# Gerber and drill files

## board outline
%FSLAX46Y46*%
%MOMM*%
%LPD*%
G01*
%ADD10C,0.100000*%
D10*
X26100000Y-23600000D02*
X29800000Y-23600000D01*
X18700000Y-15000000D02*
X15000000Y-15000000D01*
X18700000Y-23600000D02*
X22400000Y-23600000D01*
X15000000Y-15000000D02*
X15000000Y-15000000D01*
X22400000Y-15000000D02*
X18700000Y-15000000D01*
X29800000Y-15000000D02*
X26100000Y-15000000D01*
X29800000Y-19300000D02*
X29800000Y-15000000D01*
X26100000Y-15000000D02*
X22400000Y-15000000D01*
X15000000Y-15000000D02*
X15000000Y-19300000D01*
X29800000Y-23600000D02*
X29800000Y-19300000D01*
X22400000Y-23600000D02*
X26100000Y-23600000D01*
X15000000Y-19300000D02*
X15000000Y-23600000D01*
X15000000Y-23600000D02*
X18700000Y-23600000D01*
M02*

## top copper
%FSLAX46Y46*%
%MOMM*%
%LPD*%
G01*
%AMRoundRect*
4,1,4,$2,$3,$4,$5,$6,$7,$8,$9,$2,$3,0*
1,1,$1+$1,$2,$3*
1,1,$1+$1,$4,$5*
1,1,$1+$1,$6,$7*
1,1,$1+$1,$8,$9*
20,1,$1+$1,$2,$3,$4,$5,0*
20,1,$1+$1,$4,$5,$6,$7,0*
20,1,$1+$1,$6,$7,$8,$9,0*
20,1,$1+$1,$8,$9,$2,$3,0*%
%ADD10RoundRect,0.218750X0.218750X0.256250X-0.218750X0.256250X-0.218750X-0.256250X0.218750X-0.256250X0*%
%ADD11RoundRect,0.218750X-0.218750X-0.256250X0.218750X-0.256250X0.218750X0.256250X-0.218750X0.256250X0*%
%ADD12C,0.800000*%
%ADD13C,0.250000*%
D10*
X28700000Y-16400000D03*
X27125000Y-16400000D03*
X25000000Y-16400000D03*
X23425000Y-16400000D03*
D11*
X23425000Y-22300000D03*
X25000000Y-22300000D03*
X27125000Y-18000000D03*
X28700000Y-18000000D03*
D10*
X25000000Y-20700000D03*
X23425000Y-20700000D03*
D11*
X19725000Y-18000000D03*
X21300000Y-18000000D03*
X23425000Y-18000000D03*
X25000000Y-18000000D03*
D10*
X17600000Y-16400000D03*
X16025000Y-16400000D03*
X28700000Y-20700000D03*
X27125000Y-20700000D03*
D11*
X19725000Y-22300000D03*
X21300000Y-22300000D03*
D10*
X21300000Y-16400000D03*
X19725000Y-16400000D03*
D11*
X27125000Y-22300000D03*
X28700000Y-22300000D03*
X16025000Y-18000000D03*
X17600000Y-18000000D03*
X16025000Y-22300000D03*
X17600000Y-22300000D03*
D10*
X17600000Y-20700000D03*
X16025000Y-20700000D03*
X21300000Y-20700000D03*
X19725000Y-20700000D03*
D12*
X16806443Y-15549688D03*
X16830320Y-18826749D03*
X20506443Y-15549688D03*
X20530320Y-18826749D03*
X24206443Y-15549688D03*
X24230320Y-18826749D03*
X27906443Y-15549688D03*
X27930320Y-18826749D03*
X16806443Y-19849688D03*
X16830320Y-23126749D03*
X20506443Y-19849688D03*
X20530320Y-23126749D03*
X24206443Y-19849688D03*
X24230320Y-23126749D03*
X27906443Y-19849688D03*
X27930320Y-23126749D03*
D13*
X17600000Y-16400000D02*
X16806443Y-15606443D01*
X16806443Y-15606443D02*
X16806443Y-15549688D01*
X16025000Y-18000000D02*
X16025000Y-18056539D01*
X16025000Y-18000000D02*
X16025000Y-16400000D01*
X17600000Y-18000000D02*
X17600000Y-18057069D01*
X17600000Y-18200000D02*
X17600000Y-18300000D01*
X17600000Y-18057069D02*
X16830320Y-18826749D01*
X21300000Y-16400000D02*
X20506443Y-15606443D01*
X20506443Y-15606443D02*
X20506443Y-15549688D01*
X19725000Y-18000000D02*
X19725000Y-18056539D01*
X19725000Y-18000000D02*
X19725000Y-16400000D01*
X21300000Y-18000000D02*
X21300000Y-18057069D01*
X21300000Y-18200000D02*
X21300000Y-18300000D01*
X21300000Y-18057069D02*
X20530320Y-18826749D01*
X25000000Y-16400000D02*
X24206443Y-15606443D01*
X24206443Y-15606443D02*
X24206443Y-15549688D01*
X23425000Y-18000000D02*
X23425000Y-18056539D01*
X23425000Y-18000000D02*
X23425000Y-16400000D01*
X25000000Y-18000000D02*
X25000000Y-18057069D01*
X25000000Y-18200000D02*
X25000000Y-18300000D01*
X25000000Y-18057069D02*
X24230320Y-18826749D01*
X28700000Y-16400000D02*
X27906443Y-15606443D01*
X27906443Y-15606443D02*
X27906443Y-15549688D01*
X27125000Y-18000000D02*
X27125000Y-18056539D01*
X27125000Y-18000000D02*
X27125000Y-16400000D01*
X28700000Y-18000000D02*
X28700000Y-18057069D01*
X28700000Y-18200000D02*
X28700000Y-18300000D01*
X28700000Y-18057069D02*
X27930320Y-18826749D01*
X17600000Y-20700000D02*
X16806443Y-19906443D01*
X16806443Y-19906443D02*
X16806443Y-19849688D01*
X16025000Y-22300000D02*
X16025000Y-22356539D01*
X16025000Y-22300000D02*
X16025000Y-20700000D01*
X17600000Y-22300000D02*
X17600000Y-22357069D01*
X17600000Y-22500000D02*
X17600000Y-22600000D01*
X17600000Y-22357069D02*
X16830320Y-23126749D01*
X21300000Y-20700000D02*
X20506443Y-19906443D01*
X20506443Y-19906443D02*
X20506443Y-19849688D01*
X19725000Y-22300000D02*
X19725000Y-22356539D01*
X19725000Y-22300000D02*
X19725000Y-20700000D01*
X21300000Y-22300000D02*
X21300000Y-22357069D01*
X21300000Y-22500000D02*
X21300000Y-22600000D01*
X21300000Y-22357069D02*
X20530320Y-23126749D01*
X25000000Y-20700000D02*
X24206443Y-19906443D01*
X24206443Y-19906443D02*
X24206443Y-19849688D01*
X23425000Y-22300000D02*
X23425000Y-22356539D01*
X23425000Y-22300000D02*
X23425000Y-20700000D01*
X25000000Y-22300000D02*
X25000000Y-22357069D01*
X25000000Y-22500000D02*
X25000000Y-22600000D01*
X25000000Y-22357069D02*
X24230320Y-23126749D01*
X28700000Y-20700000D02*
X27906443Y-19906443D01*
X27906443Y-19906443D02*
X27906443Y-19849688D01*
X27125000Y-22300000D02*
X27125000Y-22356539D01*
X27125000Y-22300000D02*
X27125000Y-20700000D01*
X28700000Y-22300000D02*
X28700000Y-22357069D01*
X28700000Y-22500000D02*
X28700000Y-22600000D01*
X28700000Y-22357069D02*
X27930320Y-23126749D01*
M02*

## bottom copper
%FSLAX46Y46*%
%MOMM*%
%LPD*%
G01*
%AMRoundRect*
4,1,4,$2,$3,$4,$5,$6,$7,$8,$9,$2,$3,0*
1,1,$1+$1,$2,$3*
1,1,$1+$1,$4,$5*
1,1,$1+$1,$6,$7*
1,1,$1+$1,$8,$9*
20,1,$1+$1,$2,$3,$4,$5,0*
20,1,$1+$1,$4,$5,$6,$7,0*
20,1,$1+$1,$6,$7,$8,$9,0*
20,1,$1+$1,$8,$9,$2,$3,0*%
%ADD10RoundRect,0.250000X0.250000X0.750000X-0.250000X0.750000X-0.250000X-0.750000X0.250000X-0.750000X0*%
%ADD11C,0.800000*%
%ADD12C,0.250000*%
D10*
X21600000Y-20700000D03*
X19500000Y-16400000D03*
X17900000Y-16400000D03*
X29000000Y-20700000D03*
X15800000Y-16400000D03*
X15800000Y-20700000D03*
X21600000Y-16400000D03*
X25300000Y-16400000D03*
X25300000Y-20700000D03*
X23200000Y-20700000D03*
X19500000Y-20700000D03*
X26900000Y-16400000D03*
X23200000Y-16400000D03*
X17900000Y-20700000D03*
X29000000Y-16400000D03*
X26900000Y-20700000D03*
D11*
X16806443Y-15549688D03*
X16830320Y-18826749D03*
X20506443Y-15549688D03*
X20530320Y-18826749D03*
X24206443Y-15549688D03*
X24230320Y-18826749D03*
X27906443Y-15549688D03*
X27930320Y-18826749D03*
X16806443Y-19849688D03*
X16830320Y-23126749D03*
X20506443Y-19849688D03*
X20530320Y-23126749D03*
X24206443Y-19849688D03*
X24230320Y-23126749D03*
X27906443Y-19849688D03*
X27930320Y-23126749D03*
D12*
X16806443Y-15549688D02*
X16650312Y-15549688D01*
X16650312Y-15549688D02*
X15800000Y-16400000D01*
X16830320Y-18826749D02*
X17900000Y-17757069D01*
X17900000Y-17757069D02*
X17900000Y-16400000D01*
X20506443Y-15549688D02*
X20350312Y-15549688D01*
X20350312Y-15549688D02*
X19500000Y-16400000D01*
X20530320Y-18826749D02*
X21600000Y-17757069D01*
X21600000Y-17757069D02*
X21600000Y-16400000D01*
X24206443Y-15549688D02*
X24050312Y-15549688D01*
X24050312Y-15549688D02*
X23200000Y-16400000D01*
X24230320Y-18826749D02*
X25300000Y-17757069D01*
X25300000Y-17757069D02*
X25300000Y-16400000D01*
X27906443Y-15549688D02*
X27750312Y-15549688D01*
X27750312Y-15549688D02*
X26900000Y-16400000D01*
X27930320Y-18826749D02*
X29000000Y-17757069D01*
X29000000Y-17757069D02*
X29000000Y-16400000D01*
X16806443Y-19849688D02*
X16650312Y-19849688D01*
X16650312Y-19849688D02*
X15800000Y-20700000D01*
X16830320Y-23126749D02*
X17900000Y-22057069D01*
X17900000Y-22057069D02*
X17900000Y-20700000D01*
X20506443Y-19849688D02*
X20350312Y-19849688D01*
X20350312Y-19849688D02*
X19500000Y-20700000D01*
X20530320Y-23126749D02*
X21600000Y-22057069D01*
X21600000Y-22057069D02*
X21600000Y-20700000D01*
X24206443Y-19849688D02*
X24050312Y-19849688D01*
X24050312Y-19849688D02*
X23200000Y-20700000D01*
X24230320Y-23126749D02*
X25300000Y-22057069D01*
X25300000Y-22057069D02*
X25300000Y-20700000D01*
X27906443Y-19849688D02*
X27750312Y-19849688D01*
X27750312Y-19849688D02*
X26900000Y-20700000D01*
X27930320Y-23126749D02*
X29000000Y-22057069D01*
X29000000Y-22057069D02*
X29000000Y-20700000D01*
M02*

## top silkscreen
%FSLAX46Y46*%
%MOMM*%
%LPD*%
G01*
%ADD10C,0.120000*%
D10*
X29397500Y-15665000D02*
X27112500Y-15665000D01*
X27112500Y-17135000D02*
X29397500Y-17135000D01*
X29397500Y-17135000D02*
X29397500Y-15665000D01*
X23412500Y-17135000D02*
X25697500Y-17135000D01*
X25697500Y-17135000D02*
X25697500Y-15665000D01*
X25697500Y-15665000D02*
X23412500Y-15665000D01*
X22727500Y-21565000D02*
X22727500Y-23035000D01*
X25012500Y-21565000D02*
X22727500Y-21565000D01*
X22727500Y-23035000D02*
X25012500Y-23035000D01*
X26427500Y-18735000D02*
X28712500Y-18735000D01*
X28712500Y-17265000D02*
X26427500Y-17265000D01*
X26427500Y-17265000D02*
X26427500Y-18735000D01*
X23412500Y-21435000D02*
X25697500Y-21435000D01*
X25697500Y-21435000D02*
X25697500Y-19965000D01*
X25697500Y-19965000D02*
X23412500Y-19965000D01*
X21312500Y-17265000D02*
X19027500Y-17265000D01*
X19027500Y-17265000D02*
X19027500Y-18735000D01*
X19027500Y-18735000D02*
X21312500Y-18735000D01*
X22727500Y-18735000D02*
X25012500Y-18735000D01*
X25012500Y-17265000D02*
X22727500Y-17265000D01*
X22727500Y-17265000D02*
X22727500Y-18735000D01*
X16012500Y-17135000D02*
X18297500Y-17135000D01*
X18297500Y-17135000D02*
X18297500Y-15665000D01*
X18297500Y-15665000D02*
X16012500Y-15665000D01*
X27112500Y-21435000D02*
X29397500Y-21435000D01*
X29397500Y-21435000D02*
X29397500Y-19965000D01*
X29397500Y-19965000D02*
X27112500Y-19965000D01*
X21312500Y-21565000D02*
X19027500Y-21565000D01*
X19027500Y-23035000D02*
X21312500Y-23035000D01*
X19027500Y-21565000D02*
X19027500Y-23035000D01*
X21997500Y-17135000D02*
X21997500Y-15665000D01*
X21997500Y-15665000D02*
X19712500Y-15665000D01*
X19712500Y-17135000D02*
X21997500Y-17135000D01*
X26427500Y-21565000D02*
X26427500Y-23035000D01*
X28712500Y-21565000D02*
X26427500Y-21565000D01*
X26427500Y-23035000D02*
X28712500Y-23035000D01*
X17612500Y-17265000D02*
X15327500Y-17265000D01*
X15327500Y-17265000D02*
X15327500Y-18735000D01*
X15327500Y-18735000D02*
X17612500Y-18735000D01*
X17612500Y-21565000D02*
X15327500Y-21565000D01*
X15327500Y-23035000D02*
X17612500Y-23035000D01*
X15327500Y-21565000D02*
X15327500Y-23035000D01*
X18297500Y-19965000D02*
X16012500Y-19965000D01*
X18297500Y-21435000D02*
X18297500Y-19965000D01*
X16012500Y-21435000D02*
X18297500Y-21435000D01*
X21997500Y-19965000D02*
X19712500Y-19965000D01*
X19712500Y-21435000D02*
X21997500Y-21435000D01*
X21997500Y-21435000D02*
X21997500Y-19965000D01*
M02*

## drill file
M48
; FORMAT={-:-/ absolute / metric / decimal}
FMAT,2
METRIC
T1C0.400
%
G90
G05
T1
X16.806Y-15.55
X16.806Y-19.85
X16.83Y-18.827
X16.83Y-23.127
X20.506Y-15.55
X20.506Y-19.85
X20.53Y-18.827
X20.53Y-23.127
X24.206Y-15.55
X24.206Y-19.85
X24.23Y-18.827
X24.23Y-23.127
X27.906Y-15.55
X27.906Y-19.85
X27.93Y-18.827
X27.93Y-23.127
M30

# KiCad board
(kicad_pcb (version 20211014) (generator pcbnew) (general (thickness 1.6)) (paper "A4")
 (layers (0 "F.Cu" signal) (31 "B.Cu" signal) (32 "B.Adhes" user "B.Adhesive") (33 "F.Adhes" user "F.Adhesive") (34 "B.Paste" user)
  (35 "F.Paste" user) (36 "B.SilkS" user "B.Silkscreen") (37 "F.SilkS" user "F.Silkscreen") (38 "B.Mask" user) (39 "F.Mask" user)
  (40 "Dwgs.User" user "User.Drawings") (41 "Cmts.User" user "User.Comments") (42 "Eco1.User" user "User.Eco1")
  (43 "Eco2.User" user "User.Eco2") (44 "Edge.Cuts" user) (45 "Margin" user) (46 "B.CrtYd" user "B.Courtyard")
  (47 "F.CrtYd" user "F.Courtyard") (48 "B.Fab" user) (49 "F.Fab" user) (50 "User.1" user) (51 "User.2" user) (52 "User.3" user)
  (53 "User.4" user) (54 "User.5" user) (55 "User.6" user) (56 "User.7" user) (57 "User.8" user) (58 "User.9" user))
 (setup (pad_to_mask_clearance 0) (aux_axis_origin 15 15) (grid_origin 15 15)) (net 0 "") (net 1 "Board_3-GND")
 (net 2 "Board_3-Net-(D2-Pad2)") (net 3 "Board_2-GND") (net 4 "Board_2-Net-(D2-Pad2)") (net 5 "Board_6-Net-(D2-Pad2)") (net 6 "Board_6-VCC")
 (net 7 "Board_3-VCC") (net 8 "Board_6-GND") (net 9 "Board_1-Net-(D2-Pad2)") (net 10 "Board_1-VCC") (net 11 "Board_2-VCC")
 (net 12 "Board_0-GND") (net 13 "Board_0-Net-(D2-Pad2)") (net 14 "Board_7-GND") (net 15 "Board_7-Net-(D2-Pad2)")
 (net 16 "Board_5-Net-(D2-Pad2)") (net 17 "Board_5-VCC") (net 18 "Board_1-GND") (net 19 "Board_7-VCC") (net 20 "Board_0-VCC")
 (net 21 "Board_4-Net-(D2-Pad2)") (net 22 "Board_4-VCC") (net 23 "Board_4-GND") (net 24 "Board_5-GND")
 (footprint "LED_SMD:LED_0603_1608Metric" (layer "F.Cu") (at 27.9125 16.4 180)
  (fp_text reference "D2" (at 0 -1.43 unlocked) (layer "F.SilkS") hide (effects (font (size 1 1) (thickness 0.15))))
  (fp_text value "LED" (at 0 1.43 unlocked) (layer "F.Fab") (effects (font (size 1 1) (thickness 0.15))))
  (fp_line (start -1.485 0.735) (end 0.8 0.735) (layer "F.SilkS") (width 0.12))
  (fp_line (start 0.8 -0.735) (end -1.485 -0.735) (layer "F.SilkS") (width 0.12))
  (fp_line (start -1.485 -0.735) (end -1.485 0.735) (layer "F.SilkS") (width 0.12))
  (pad "1" smd roundrect (at -0.7875 0 180) (size 0.875 0.95) (layers "F.Cu" "F.Paste" "F.Mask") (roundrect_rratio 0.25)
   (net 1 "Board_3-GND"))
  (pad "2" smd roundrect (at 0.7875 0 180) (size 0.875 0.95) (layers "F.Cu" "F.Paste" "F.Mask") (roundrect_rratio 0.25)
   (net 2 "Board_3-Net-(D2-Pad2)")))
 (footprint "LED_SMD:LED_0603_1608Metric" (layer "F.Cu") (at 24.2125 16.4 180)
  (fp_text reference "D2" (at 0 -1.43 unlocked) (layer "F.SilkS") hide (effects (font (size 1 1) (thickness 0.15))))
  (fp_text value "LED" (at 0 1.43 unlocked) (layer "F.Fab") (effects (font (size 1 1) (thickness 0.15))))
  (fp_line (start 0.8 -0.735) (end -1.485 -0.735) (layer "F.SilkS") (width 0.12))
  (fp_line (start -1.485 -0.735) (end -1.485 0.735) (layer "F.SilkS") (width 0.12))
  (fp_line (start -1.485 0.735) (end 0.8 0.735) (layer "F.SilkS") (width 0.12))
  (pad "1" smd roundrect (at -0.7875 0 180) (size 0.875 0.95) (layers "F.Cu" "F.Paste" "F.Mask") (roundrect_rratio 0.25)
   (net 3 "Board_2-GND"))
  (pad "2" smd roundrect (at 0.7875 0 180) (size 0.875 0.95) (layers "F.Cu" "F.Paste" "F.Mask") (roundrect_rratio 0.25)
   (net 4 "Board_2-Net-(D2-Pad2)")))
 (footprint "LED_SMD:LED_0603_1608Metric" (layer "F.Cu") (at 24.2125 22.3)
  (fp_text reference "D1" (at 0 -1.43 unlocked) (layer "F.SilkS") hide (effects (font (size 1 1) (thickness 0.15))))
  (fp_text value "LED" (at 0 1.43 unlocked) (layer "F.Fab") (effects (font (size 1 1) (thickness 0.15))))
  (fp_line (start -1.485 -0.735) (end -1.485 0.735) (layer "F.SilkS") (width 0.12))
  (fp_line (start 0.8 -0.735) (end -1.485 -0.735) (layer "F.SilkS") (width 0.12))
  (fp_line (start -1.485 0.735) (end 0.8 0.735) (layer "F.SilkS") (width 0.12))
  (pad "1" smd roundrect (at -0.7875 0) (size 0.875 0.95) (layers "F.Cu" "F.Paste" "F.Mask") (roundrect_rratio 0.25)
   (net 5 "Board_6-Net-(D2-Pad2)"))
  (pad "2" smd roundrect (at 0.7875 0) (size 0.875 0.95) (layers "F.Cu" "F.Paste" "F.Mask") (roundrect_rratio 0.25) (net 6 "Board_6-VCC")))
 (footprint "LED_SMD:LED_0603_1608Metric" (layer "F.Cu") (at 27.9125 18)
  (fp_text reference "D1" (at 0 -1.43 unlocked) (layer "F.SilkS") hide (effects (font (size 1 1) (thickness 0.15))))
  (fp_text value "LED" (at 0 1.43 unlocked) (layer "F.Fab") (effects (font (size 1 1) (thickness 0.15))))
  (fp_line (start -1.485 0.735) (end 0.8 0.735) (layer "F.SilkS") (width 0.12))
  (fp_line (start 0.8 -0.735) (end -1.485 -0.735) (layer "F.SilkS") (width 0.12))
  (fp_line (start -1.485 -0.735) (end -1.485 0.735) (layer "F.SilkS") (width 0.12))
  (pad "1" smd roundrect (at -0.7875 0) (size 0.875 0.95) (layers "F.Cu" "F.Paste" "F.Mask") (roundrect_rratio 0.25)
   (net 2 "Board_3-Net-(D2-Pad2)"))
  (pad "2" smd roundrect (at 0.7875 0) (size 0.875 0.95) (layers "F.Cu" "F.Paste" "F.Mask") (roundrect_rratio 0.25) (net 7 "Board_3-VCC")))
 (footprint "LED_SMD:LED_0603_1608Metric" (layer "F.Cu") (at 24.2125 20.7 180)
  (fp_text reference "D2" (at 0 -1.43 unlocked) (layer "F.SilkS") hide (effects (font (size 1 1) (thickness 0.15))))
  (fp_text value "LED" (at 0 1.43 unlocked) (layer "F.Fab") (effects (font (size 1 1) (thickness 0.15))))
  (fp_line (start 0.8 -0.735) (end -1.485 -0.735) (layer "F.SilkS") (width 0.12))
  (fp_line (start -1.485 -0.735) (end -1.485 0.735) (layer "F.SilkS") (width 0.12))
  (fp_line (start -1.485 0.735) (end 0.8 0.735) (layer "F.SilkS") (width 0.12))
  (pad "1" smd roundrect (at -0.7875 0 180) (size 0.875 0.95) (layers "F.Cu" "F.Paste" "F.Mask") (roundrect_rratio 0.25)
   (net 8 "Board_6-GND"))
  (pad "2" smd roundrect (at 0.7875 0 180) (size 0.875 0.95) (layers "F.Cu" "F.Paste" "F.Mask") (roundrect_rratio 0.25)
   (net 5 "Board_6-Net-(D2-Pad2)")))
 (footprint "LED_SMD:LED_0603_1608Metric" (layer "F.Cu") (at 20.5125 18)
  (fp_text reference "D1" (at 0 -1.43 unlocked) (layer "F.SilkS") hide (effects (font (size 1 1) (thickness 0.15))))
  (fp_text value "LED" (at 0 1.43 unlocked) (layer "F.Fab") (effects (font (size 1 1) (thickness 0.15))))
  (fp_line (start 0.8 -0.735) (end -1.485 -0.735) (layer "F.SilkS") (width 0.12))
  (fp_line (start -1.485 -0.735) (end -1.485 0.735) (layer "F.SilkS") (width 0.12))
  (fp_line (start -1.485 0.735) (end 0.8 0.735) (layer "F.SilkS") (width 0.12))
  (pad "1" smd roundrect (at -0.7875 0) (size 0.875 0.95) (layers "F.Cu" "F.Paste" "F.Mask") (roundrect_rratio 0.25)
   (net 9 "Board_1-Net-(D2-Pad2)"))
  (pad "2" smd roundrect (at 0.7875 0) (size 0.875 0.95) (layers "F.Cu" "F.Paste" "F.Mask") (roundrect_rratio 0.25) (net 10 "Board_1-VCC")))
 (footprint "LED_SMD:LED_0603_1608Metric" (layer "F.Cu") (at 24.2125 18)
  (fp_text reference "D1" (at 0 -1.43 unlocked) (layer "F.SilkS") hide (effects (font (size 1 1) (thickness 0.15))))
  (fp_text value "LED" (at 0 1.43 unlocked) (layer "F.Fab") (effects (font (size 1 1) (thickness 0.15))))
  (fp_line (start -1.485 0.735) (end 0.8 0.735) (layer "F.SilkS") (width 0.12))
  (fp_line (start 0.8 -0.735) (end -1.485 -0.735) (layer "F.SilkS") (width 0.12))
  (fp_line (start -1.485 -0.735) (end -1.485 0.735) (layer "F.SilkS") (width 0.12))
  (pad "1" smd roundrect (at -0.7875 0) (size 0.875 0.95) (layers "F.Cu" "F.Paste" "F.Mask") (roundrect_rratio 0.25)
   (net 4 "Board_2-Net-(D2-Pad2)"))
  (pad "2" smd roundrect (at 0.7875 0) (size 0.875 0.95) (layers "F.Cu" "F.Paste" "F.Mask") (roundrect_rratio 0.25) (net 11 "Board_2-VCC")))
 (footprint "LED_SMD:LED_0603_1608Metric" (layer "F.Cu") (at 16.8125 16.4 180)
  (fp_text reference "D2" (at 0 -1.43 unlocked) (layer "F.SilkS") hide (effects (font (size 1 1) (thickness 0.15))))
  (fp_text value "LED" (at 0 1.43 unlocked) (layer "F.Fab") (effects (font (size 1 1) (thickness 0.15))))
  (fp_line (start 0.8 -0.735) (end -1.485 -0.735) (layer "F.SilkS") (width 0.12))
  (fp_line (start -1.485 -0.735) (end -1.485 0.735) (layer "F.SilkS") (width 0.12))
  (fp_line (start -1.485 0.735) (end 0.8 0.735) (layer "F.SilkS") (width 0.12))
  (pad "1" smd roundrect (at -0.7875 0 180) (size 0.875 0.95) (layers "F.Cu" "F.Paste" "F.Mask") (roundrect_rratio 0.25)
   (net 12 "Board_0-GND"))
  (pad "2" smd roundrect (at 0.7875 0 180) (size 0.875 0.95) (layers "F.Cu" "F.Paste" "F.Mask") (roundrect_rratio 0.25)
   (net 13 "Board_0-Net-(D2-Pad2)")))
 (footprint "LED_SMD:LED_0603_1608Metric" (layer "F.Cu") (at 27.9125 20.7 180)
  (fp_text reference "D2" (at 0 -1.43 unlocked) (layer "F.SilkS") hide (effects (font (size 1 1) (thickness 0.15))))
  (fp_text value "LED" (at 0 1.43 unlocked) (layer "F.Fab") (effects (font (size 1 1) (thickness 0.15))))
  (fp_line (start 0.8 -0.735) (end -1.485 -0.735) (layer "F.SilkS") (width 0.12))
  (fp_line (start -1.485 -0.735) (end -1.485 0.735) (layer "F.SilkS") (width 0.12))
  (fp_line (start -1.485 0.735) (end 0.8 0.735) (layer "F.SilkS") (width 0.12))
  (pad "1" smd roundrect (at -0.7875 0 180) (size 0.875 0.95) (layers "F.Cu" "F.Paste" "F.Mask") (roundrect_rratio 0.25)
   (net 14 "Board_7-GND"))
  (pad "2" smd roundrect (at 0.7875 0 180) (size 0.875 0.95) (layers "F.Cu" "F.Paste" "F.Mask") (roundrect_rratio 0.25)
   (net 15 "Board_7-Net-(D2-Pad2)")))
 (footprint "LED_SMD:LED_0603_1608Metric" (layer "F.Cu") (at 20.5125 22.3)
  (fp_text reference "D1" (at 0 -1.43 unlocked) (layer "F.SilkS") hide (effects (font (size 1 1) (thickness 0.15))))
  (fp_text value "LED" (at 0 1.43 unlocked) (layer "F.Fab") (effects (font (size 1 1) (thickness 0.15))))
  (fp_line (start 0.8 -0.735) (end -1.485 -0.735) (layer "F.SilkS") (width 0.12))
  (fp_line (start -1.485 0.735) (end 0.8 0.735) (layer "F.SilkS") (width 0.12))
  (fp_line (start -1.485 -0.735) (end -1.485 0.735) (layer "F.SilkS") (width 0.12))
  (pad "1" smd roundrect (at -0.7875 0) (size 0.875 0.95) (layers "F.Cu" "F.Paste" "F.Mask") (roundrect_rratio 0.25)
   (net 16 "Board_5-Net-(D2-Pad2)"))
  (pad "2" smd roundrect (at 0.7875 0) (size 0.875 0.95) (layers "F.Cu" "F.Paste" "F.Mask") (roundrect_rratio 0.25) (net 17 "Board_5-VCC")))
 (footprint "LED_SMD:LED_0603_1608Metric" (layer "F.Cu") (at 20.5125 16.4 180)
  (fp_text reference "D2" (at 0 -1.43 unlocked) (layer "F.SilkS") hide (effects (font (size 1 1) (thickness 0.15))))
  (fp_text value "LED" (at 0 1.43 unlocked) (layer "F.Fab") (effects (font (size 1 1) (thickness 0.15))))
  (fp_line (start -1.485 -0.735) (end -1.485 0.735) (layer "F.SilkS") (width 0.12))
  (fp_line (start -1.485 0.735) (end 0.8 0.735) (layer "F.SilkS") (width 0.12))
  (fp_line (start 0.8 -0.735) (end -1.485 -0.735) (layer "F.SilkS") (width 0.12))
  (pad "1" smd roundrect (at -0.7875 0 180) (size 0.875 0.95) (layers "F.Cu" "F.Paste" "F.Mask") (roundrect_rratio 0.25)
   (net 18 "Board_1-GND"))
  (pad "2" smd roundrect (at 0.7875 0 180) (size 0.875 0.95) (layers "F.Cu" "F.Paste" "F.Mask") (roundrect_rratio 0.25)
   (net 9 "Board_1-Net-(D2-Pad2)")))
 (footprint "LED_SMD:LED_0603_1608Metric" (layer "F.Cu") (at 27.9125 22.3)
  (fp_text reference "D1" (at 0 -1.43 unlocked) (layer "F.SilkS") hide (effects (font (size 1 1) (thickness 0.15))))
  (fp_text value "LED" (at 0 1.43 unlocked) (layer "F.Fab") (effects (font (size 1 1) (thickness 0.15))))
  (fp_line (start -1.485 -0.735) (end -1.485 0.735) (layer "F.SilkS") (width 0.12))
  (fp_line (start 0.8 -0.735) (end -1.485 -0.735) (layer "F.SilkS") (width 0.12))
  (fp_line (start -1.485 0.735) (end 0.8 0.735) (layer "F.SilkS") (width 0.12))
  (pad "1" smd roundrect (at -0.7875 0) (size 0.875 0.95) (layers "F.Cu" "F.Paste" "F.Mask") (roundrect_rratio 0.25)
   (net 15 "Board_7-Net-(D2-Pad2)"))
  (pad "2" smd roundrect (at 0.7875 0) (size 0.875 0.95) (layers "F.Cu" "F.Paste" "F.Mask") (roundrect_rratio 0.25) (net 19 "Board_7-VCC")))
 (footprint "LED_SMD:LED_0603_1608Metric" (layer "F.Cu") (at 16.8125 18)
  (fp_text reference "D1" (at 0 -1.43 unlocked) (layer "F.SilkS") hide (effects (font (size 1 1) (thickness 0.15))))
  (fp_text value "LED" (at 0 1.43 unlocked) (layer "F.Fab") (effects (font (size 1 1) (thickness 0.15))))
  (fp_line (start 0.8 -0.735) (end -1.485 -0.735) (layer "F.SilkS") (width 0.12))
  (fp_line (start -1.485 -0.735) (end -1.485 0.735) (layer "F.SilkS") (width 0.12))
  (fp_line (start -1.485 0.735) (end 0.8 0.735) (layer "F.SilkS") (width 0.12))
  (pad "1" smd roundrect (at -0.7875 0) (size 0.875 0.95) (layers "F.Cu" "F.Paste" "F.Mask") (roundrect_rratio 0.25)
   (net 13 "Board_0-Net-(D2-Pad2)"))
  (pad "2" smd roundrect (at 0.7875 0) (size 0.875 0.95) (layers "F.Cu" "F.Paste" "F.Mask") (roundrect_rratio 0.25) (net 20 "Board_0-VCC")))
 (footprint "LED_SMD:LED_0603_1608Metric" (layer "F.Cu") (at 16.8125 22.3)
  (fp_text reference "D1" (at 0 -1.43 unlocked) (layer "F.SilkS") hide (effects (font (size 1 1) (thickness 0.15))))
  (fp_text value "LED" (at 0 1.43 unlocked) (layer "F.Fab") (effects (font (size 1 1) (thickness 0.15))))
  (fp_line (start 0.8 -0.735) (end -1.485 -0.735) (layer "F.SilkS") (width 0.12))
  (fp_line (start -1.485 0.735) (end 0.8 0.735) (layer "F.SilkS") (width 0.12))
  (fp_line (start -1.485 -0.735) (end -1.485 0.735) (layer "F.SilkS") (width 0.12))
  (pad "1" smd roundrect (at -0.7875 0) (size 0.875 0.95) (layers "F.Cu" "F.Paste" "F.Mask") (roundrect_rratio 0.25)
   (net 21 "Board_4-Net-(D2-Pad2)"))
  (pad "2" smd roundrect (at 0.7875 0) (size 0.875 0.95) (layers "F.Cu" "F.Paste" "F.Mask") (roundrect_rratio 0.25) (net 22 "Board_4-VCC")))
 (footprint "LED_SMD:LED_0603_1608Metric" (layer "F.Cu") (at 16.8125 20.7 180)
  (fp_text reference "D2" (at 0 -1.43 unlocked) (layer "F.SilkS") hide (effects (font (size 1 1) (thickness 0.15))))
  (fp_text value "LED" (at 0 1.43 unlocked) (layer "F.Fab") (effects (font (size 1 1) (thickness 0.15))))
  (fp_line (start -1.485 0.735) (end 0.8 0.735) (layer "F.SilkS") (width 0.12))
  (fp_line (start -1.485 -0.735) (end -1.485 0.735) (layer "F.SilkS") (width 0.12))
  (fp_line (start 0.8 -0.735) (end -1.485 -0.735) (layer "F.SilkS") (width 0.12))
  (pad "1" smd roundrect (at -0.7875 0 180) (size 0.875 0.95) (layers "F.Cu" "F.Paste" "F.Mask") (roundrect_rratio 0.25)
   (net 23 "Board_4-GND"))
  (pad "2" smd roundrect (at 0.7875 0 180) (size 0.875 0.95) (layers "F.Cu" "F.Paste" "F.Mask") (roundrect_rratio 0.25)
   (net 21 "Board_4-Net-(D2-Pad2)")))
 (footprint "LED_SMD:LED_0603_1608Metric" (layer "F.Cu") (at 20.5125 20.7 180)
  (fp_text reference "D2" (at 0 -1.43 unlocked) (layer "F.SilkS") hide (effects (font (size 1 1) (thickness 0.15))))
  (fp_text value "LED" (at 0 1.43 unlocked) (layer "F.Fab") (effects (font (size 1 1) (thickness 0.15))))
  (fp_line (start -1.485 0.735) (end 0.8 0.735) (layer "F.SilkS") (width 0.12))
  (fp_line (start 0.8 -0.735) (end -1.485 -0.735) (layer "F.SilkS") (width 0.12))
  (fp_line (start -1.485 -0.735) (end -1.485 0.735) (layer "F.SilkS") (width 0.12))
  (pad "1" smd roundrect (at -0.7875 0 180) (size 0.875 0.95) (layers "F.Cu" "F.Paste" "F.Mask") (roundrect_rratio 0.25)
   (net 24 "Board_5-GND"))
  (pad "2" smd roundrect (at 0.7875 0 180) (size 0.875 0.95) (layers "F.Cu" "F.Paste" "F.Mask") (roundrect_rratio 0.25)
   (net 16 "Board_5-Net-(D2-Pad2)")))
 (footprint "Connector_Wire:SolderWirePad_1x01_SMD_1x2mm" (layer "B.Cu") (at 21.6 20.7 180)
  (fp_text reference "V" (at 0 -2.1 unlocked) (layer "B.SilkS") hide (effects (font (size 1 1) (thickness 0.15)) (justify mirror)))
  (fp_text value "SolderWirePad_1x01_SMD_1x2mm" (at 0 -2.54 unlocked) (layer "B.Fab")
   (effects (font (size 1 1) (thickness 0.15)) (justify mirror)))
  (pad "1" smd roundrect (at 0 0 180) (size 1 2) (layers "B.Cu" "B.Paste" "B.Mask") (roundrect_rratio 0.25) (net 17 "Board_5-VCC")))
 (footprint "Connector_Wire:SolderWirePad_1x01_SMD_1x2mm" (layer "B.Cu") (at 19.5 16.4 180)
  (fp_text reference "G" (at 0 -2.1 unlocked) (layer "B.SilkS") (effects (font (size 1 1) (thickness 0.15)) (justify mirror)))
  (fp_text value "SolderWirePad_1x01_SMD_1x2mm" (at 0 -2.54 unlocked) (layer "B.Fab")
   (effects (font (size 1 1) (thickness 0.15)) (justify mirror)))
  (pad "1" smd roundrect (at 0 0 180) (size 1 2) (layers "B.Cu" "B.Paste" "B.Mask") (roundrect_rratio 0.25) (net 18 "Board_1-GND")))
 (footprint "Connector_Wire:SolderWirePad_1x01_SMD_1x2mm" (layer "B.Cu") (at 17.9 16.4 180)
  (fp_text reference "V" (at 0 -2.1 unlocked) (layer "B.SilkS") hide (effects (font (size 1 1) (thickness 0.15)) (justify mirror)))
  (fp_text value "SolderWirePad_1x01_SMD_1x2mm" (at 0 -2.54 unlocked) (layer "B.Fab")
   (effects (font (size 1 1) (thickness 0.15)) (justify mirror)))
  (pad "1" smd roundrect (at 0 0 180) (size 1 2) (layers "B.Cu" "B.Paste" "B.Mask") (roundrect_rratio 0.25) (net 20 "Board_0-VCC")))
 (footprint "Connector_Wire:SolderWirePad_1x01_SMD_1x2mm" (layer "B.Cu") (at 29 20.7 180)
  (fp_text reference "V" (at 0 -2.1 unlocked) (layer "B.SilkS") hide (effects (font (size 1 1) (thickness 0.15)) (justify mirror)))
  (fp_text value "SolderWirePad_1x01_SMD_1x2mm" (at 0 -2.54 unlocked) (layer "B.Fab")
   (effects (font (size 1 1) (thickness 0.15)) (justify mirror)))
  (pad "1" smd roundrect (at 0 0 180) (size 1 2) (layers "B.Cu" "B.Paste" "B.Mask") (roundrect_rratio 0.25) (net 19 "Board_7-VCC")))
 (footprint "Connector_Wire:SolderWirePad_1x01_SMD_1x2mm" (layer "B.Cu") (at 15.8 16.4 180)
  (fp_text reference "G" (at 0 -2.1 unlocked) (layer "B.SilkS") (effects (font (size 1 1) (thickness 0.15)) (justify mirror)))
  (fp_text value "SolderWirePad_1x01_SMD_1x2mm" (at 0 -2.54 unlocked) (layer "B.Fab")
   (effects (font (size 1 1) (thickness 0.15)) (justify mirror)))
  (pad "1" smd roundrect (at 0 0 180) (size 1 2) (layers "B.Cu" "B.Paste" "B.Mask") (roundrect_rratio 0.25) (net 12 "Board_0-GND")))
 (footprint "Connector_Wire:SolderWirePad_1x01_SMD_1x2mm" (layer "B.Cu") (at 15.8 20.7 180)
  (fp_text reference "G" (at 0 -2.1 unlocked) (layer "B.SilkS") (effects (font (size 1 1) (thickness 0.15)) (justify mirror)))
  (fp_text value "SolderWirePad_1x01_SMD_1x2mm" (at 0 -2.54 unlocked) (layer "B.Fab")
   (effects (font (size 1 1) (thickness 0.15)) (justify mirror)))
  (pad "1" smd roundrect (at 0 0 180) (size 1 2) (layers "B.Cu" "B.Paste" "B.Mask") (roundrect_rratio 0.25) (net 23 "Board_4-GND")))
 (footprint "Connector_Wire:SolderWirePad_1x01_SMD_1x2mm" (layer "B.Cu") (at 21.6 16.4 180)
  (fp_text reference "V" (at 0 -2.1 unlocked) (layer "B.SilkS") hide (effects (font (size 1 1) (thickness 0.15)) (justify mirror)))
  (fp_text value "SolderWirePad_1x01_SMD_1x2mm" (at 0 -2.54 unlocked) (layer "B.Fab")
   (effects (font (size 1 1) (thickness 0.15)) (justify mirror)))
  (pad "1" smd roundrect (at 0 0 180) (size 1 2) (layers "B.Cu" "B.Paste" "B.Mask") (roundrect_rratio 0.25) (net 10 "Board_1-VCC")))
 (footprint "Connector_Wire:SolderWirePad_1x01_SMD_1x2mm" (layer "B.Cu") (at 25.3 16.4 180)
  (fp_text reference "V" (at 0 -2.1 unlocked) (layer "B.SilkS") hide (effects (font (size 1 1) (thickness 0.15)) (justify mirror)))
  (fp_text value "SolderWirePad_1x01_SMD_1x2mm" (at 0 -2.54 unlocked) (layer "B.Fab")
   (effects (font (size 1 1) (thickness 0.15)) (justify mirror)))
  (pad "1" smd roundrect (at 0 0 180) (size 1 2) (layers "B.Cu" "B.Paste" "B.Mask") (roundrect_rratio 0.25) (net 11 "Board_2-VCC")))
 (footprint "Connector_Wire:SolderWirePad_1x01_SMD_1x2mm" (layer "B.Cu") (at 25.3 20.7 180)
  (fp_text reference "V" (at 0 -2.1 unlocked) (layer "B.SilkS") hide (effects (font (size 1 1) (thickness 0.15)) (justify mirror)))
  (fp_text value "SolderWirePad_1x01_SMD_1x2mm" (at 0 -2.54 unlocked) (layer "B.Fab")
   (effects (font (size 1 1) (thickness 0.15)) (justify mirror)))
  (pad "1" smd roundrect (at 0 0 180) (size 1 2) (layers "B.Cu" "B.Paste" "B.Mask") (roundrect_rratio 0.25) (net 6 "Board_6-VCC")))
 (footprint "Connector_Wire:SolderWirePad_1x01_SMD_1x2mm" (layer "B.Cu") (at 23.2 20.7 180)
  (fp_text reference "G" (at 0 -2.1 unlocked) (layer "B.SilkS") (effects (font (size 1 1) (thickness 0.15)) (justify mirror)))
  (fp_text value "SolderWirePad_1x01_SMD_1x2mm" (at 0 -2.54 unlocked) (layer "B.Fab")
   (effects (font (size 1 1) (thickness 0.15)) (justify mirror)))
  (pad "1" smd roundrect (at 0 0 180) (size 1 2) (layers "B.Cu" "B.Paste" "B.Mask") (roundrect_rratio 0.25) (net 8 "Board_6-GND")))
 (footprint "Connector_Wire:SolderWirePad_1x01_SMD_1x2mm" (layer "B.Cu") (at 19.5 20.7 180)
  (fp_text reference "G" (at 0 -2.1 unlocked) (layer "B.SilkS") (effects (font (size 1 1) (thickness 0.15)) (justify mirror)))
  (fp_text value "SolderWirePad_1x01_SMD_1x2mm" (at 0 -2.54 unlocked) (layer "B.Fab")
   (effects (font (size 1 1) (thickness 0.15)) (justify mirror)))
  (pad "1" smd roundrect (at 0 0 180) (size 1 2) (layers "B.Cu" "B.Paste" "B.Mask") (roundrect_rratio 0.25) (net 24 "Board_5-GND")))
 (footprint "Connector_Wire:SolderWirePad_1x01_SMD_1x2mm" (layer "B.Cu") (at 26.9 16.4 180)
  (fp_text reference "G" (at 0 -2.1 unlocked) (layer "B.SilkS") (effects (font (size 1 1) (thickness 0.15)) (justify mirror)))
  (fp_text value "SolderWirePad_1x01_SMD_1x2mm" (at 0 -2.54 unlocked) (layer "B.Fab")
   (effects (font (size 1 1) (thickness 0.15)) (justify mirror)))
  (pad "1" smd roundrect (at 0 0 180) (size 1 2) (layers "B.Cu" "B.Paste" "B.Mask") (roundrect_rratio 0.25) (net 1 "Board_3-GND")))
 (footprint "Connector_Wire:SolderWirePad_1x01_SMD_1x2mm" (layer "B.Cu") (at 23.2 16.4 180)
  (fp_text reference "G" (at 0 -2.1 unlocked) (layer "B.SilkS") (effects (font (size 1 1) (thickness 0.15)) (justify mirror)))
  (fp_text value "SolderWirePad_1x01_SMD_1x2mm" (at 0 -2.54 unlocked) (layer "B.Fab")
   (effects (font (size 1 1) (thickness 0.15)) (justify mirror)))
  (pad "1" smd roundrect (at 0 0 180) (size 1 2) (layers "B.Cu" "B.Paste" "B.Mask") (roundrect_rratio 0.25) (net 3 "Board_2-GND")))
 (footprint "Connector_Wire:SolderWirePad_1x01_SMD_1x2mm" (layer "B.Cu") (at 17.9 20.7 180)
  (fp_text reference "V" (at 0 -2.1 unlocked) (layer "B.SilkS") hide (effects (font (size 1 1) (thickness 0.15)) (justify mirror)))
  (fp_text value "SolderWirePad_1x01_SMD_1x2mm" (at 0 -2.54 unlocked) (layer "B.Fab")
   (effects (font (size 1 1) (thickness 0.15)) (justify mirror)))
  (pad "1" smd roundrect (at 0 0 180) (size 1 2) (layers "B.Cu" "B.Paste" "B.Mask") (roundrect_rratio 0.25) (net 22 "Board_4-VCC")))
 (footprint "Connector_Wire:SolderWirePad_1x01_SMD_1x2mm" (layer "B.Cu") (at 29 16.4 180)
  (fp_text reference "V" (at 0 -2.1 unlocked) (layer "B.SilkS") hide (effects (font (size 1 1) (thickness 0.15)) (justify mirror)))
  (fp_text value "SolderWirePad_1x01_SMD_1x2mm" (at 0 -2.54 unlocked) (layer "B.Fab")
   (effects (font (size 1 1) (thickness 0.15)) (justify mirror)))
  (pad "1" smd roundrect (at 0 0 180) (size 1 2) (layers "B.Cu" "B.Paste" "B.Mask") (roundrect_rratio 0.25) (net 7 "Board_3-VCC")))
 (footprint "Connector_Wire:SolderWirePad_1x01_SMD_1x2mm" (layer "B.Cu") (at 26.9 20.7 180)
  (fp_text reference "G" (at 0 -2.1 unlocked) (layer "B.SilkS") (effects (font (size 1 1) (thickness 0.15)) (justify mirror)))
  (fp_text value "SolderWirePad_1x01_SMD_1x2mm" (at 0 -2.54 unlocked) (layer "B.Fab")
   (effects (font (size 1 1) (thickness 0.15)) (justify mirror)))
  (pad "1" smd roundrect (at 0 0 180) (size 1 2) (layers "B.Cu" "B.Paste" "B.Mask") (roundrect_rratio 0.25) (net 14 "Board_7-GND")))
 (gr_line (start 26.1 23.6) (end 29.8 23.6) (layer "Edge.Cuts") (width 0.1))
 (gr_line (start 18.7 15) (end 15 15) (layer "Edge.Cuts") (width 0.1))
 (gr_line (start 18.7 23.6) (end 22.4 23.6) (layer "Edge.Cuts") (width 0.1))
 (gr_line (start 15 15) (end 15 15) (layer "Edge.Cuts") (width 0.1))
 (gr_line (start 22.4 15) (end 18.7 15) (layer "Edge.Cuts") (width 0.1))
 (gr_line (start 29.8 15) (end 26.1 15) (layer "Edge.Cuts") (width 0.1))
 (gr_line (start 29.8 19.3) (end 29.8 15) (layer "Edge.Cuts") (width 0.1))
 (gr_line (start 26.1 15) (end 22.4 15) (layer "Edge.Cuts") (width 0.1))
 (gr_line (start 15 15) (end 15 19.3) (layer "Edge.Cuts") (width 0.1))
 (gr_line (start 29.8 23.6) (end 29.8 19.3) (layer "Edge.Cuts") (width 0.1))
 (gr_line (start 22.4 23.6) (end 26.1 23.6) (layer "Edge.Cuts") (width 0.1))
 (gr_line (start 15 19.3) (end 15 23.6) (layer "Edge.Cuts") (width 0.1))
 (gr_line (start 15 23.6) (end 18.7 23.6) (layer "Edge.Cuts") (width 0.1))
 (segment (start 17.6 16.4) (end 16.806443 15.606443) (width 0.25) (layer "F.Cu") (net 12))
 (segment (start 16.806443 15.606443) (end 16.806443 15.549688) (width 0.25) (layer "F.Cu") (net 12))
 (via (at 16.806443 15.549688) (size 0.8) (drill 0.4) (layers "F.Cu" "B.Cu") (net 12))
 (segment (start 16.806443 15.549688) (end 16.650312 15.549688) (width 0.25) (layer "B.Cu") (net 12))
 (segment (start 16.650312 15.549688) (end 15.8 16.4) (width 0.25) (layer "B.Cu") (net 12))
 (segment (start 16.025 18) (end 16.025 18.056539) (width 0.25) (layer "F.Cu") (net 13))
 (segment (start 16.025 18) (end 16.025 16.4) (width 0.25) (layer "F.Cu") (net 13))
 (segment (start 17.6 18) (end 17.6 18.057069) (width 0.25) (layer "F.Cu") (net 20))
 (segment (start 17.6 18.2) (end 17.6 18.3) (width 0.25) (layer "F.Cu") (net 20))
 (segment (start 17.6 18.057069) (end 16.83032 18.826749) (width 0.25) (layer "F.Cu") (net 20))
 (via (at 16.83032 18.826749) (size 0.8) (drill 0.4) (layers "F.Cu" "B.Cu") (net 20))
 (segment (start 16.83032 18.826749) (end 17.9 17.757069) (width 0.25) (layer "B.Cu") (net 20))
 (segment (start 17.9 17.757069) (end 17.9 16.4) (width 0.25) (layer "B.Cu") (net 20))
 (segment (start 21.3 16.4) (end 20.506443 15.606443) (width 0.25) (layer "F.Cu") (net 18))
 (segment (start 20.506443 15.606443) (end 20.506443 15.549688) (width 0.25) (layer "F.Cu") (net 18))
 (via (at 20.506443 15.549688) (size 0.8) (drill 0.4) (layers "F.Cu" "B.Cu") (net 18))
 (segment (start 20.506443 15.549688) (end 20.350312 15.549688) (width 0.25) (layer "B.Cu") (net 18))
 (segment (start 20.350312 15.549688) (end 19.5 16.4) (width 0.25) (layer "B.Cu") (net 18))
 (segment (start 19.725 18) (end 19.725 18.056539) (width 0.25) (layer "F.Cu") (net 9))
 (segment (start 19.725 18) (end 19.725 16.4) (width 0.25) (layer "F.Cu") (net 9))
 (segment (start 21.3 18) (end 21.3 18.057069) (width 0.25) (layer "F.Cu") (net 10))
 (segment (start 21.3 18.2) (end 21.3 18.3) (width 0.25) (layer "F.Cu") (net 10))
 (segment (start 21.3 18.057069) (end 20.53032 18.826749) (width 0.25) (layer "F.Cu") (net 10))
 (via (at 20.53032 18.826749) (size 0.8) (drill 0.4) (layers "F.Cu" "B.Cu") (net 10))
 (segment (start 20.53032 18.826749) (end 21.6 17.757069) (width 0.25) (layer "B.Cu") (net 10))
 (segment (start 21.6 17.757069) (end 21.6 16.4) (width 0.25) (layer "B.Cu") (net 10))
 (segment (start 25 16.4) (end 24.206443 15.606443) (width 0.25) (layer "F.Cu") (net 3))
 (segment (start 24.206443 15.606443) (end 24.206443 15.549688) (width 0.25) (layer "F.Cu") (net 3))
 (via (at 24.206443 15.549688) (size 0.8) (drill 0.4) (layers "F.Cu" "B.Cu") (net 3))
 (segment (start 24.206443 15.549688) (end 24.050312 15.549688) (width 0.25) (layer "B.Cu") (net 3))
 (segment (start 24.050312 15.549688) (end 23.2 16.4) (width 0.25) (layer "B.Cu") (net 3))
 (segment (start 23.425 18) (end 23.425 18.056539) (width 0.25) (layer "F.Cu") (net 4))
 (segment (start 23.425 18) (end 23.425 16.4) (width 0.25) (layer "F.Cu") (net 4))
 (segment (start 25 18) (end 25 18.057069) (width 0.25) (layer "F.Cu") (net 11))
 (segment (start 25 18.2) (end 25 18.3) (width 0.25) (layer "F.Cu") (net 11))
 (segment (start 25 18.057069) (end 24.23032 18.826749) (width 0.25) (layer "F.Cu") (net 11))
 (via (at 24.23032 18.826749) (size 0.8) (drill 0.4) (layers "F.Cu" "B.Cu") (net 11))
 (segment (start 24.23032 18.826749) (end 25.3 17.757069) (width 0.25) (layer "B.Cu") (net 11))
 (segment (start 25.3 17.757069) (end 25.3 16.4) (width 0.25) (layer "B.Cu") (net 11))
 (segment (start 28.7 16.4) (end 27.906443 15.606443) (width 0.25) (layer "F.Cu") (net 1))
 (segment (start 27.906443 15.606443) (end 27.906443 15.549688) (width 0.25) (layer "F.Cu") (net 1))
 (via (at 27.906443 15.549688) (size 0.8) (drill 0.4) (layers "F.Cu" "B.Cu") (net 1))
 (segment (start 27.906443 15.549688) (end 27.750312 15.549688) (width 0.25) (layer "B.Cu") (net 1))
 (segment (start 27.750312 15.549688) (end 26.9 16.4) (width 0.25) (layer "B.Cu") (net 1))
 (segment (start 27.125 18) (end 27.125 18.056539) (width 0.25) (layer "F.Cu") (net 2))
 (segment (start 27.125 18) (end 27.125 16.4) (width 0.25) (layer "F.Cu") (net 2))
 (segment (start 28.7 18) (end 28.7 18.057069) (width 0.25) (layer "F.Cu") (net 7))
 (segment (start 28.7 18.2) (end 28.7 18.3) (width 0.25) (layer "F.Cu") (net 7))
 (segment (start 28.7 18.057069) (end 27.93032 18.826749) (width 0.25) (layer "F.Cu") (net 7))
 (via (at 27.93032 18.826749) (size 0.8) (drill 0.4) (layers "F.Cu" "B.Cu") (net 7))
 (segment (start 27.93032 18.826749) (end 29 17.757069) (width 0.25) (layer "B.Cu") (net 7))
 (segment (start 29 17.757069) (end 29 16.4) (width 0.25) (layer "B.Cu") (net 7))
 (segment (start 17.6 20.7) (end 16.806443 19.906443) (width 0.25) (layer "F.Cu") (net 23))
 (segment (start 16.806443 19.906443) (end 16.806443 19.849688) (width 0.25) (layer "F.Cu") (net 23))
 (via (at 16.806443 19.849688) (size 0.8) (drill 0.4) (layers "F.Cu" "B.Cu") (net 23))
 (segment (start 16.806443 19.849688) (end 16.650312 19.849688) (width 0.25) (layer "B.Cu") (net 23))
 (segment (start 16.650312 19.849688) (end 15.8 20.7) (width 0.25) (layer "B.Cu") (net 23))
 (segment (start 16.025 22.3) (end 16.025 22.356539) (width 0.25) (layer "F.Cu") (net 21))
 (segment (start 16.025 22.3) (end 16.025 20.7) (width 0.25) (layer "F.Cu") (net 21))
 (segment (start 17.6 22.3) (end 17.6 22.357069) (width 0.25) (layer "F.Cu") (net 22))
 (segment (start 17.6 22.5) (end 17.6 22.6) (width 0.25) (layer "F.Cu") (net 22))
 (segment (start 17.6 22.357069) (end 16.83032 23.126749) (width 0.25) (layer "F.Cu") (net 22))
 (via (at 16.83032 23.126749) (size 0.8) (drill 0.4) (layers "F.Cu" "B.Cu") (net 22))
 (segment (start 16.83032 23.126749) (end 17.9 22.057069) (width 0.25) (layer "B.Cu") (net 22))
 (segment (start 17.9 22.057069) (end 17.9 20.7) (width 0.25) (layer "B.Cu") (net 22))
 (segment (start 21.3 20.7) (end 20.506443 19.906443) (width 0.25) (layer "F.Cu") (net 24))
 (segment (start 20.506443 19.906443) (end 20.506443 19.849688) (width 0.25) (layer "F.Cu") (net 24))
 (via (at 20.506443 19.849688) (size 0.8) (drill 0.4) (layers "F.Cu" "B.Cu") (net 24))
 (segment (start 20.506443 19.849688) (end 20.350312 19.849688) (width 0.25) (layer "B.Cu") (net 24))
 (segment (start 20.350312 19.849688) (end 19.5 20.7) (width 0.25) (layer "B.Cu") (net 24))
 (segment (start 19.725 22.3) (end 19.725 22.356539) (width 0.25) (layer "F.Cu") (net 16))
 (segment (start 19.725 22.3) (end 19.725 20.7) (width 0.25) (layer "F.Cu") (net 16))
 (segment (start 21.3 22.3) (end 21.3 22.357069) (width 0.25) (layer "F.Cu") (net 17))
 (segment (start 21.3 22.5) (end 21.3 22.6) (width 0.25) (layer "F.Cu") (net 17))
 (segment (start 21.3 22.357069) (end 20.53032 23.126749) (width 0.25) (layer "F.Cu") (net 17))
 (via (at 20.53032 23.126749) (size 0.8) (drill 0.4) (layers "F.Cu" "B.Cu") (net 17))
 (segment (start 20.53032 23.126749) (end 21.6 22.057069) (width 0.25) (layer "B.Cu") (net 17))
 (segment (start 21.6 22.057069) (end 21.6 20.7) (width 0.25) (layer "B.Cu") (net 17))
 (segment (start 25 20.7) (end 24.206443 19.906443) (width 0.25) (layer "F.Cu") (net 8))
 (segment (start 24.206443 19.906443) (end 24.206443 19.849688) (width 0.25) (layer "F.Cu") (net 8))
 (via (at 24.206443 19.849688) (size 0.8) (drill 0.4) (layers "F.Cu" "B.Cu") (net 8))
 (segment (start 24.206443 19.849688) (end 24.050312 19.849688) (width 0.25) (layer "B.Cu") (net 8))
 (segment (start 24.050312 19.849688) (end 23.2 20.7) (width 0.25) (layer "B.Cu") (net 8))
 (segment (start 23.425 22.3) (end 23.425 22.356539) (width 0.25) (layer "F.Cu") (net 5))
 (segment (start 23.425 22.3) (end 23.425 20.7) (width 0.25) (layer "F.Cu") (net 5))
 (segment (start 25 22.3) (end 25 22.357069) (width 0.25) (layer "F.Cu") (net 6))
 (segment (start 25 22.5) (end 25 22.6) (width 0.25) (layer "F.Cu") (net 6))
 (segment (start 25 22.357069) (end 24.23032 23.126749) (width 0.25) (layer "F.Cu") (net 6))
 (via (at 24.23032 23.126749) (size 0.8) (drill 0.4) (layers "F.Cu" "B.Cu") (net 6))
 (segment (start 24.23032 23.126749) (end 25.3 22.057069) (width 0.25) (layer "B.Cu") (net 6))
 (segment (start 25.3 22.057069) (end 25.3 20.7) (width 0.25) (layer "B.Cu") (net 6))
 (segment (start 28.7 20.7) (end 27.906443 19.906443) (width 0.25) (layer "F.Cu") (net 14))
 (segment (start 27.906443 19.906443) (end 27.906443 19.849688) (width 0.25) (layer "F.Cu") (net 14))
 (via (at 27.906443 19.849688) (size 0.8) (drill 0.4) (layers "F.Cu" "B.Cu") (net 14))
 (segment (start 27.906443 19.849688) (end 27.750312 19.849688) (width 0.25) (layer "B.Cu") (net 14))
 (segment (start 27.750312 19.849688) (end 26.9 20.7) (width 0.25) (layer "B.Cu") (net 14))
 (segment (start 27.125 22.3) (end 27.125 22.356539) (width 0.25) (layer "F.Cu") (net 15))
 (segment (start 27.125 22.3) (end 27.125 20.7) (width 0.25) (layer "F.Cu") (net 15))
 (segment (start 28.7 22.3) (end 28.7 22.357069) (width 0.25) (layer "F.Cu") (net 19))
 (segment (start 28.7 22.5) (end 28.7 22.6) (width 0.25) (layer "F.Cu") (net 19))
 (segment (start 28.7 22.357069) (end 27.93032 23.126749) (width 0.25) (layer "F.Cu") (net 19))
 (via (at 27.93032 23.126749) (size 0.8) (drill 0.4) (layers "F.Cu" "B.Cu") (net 19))
 (segment (start 27.93032 23.126749) (end 29 22.057069) (width 0.25) (layer "B.Cu") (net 19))
 (segment (start 29 22.057069) (end 29 20.7) (width 0.25) (layer "B.Cu") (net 19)))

